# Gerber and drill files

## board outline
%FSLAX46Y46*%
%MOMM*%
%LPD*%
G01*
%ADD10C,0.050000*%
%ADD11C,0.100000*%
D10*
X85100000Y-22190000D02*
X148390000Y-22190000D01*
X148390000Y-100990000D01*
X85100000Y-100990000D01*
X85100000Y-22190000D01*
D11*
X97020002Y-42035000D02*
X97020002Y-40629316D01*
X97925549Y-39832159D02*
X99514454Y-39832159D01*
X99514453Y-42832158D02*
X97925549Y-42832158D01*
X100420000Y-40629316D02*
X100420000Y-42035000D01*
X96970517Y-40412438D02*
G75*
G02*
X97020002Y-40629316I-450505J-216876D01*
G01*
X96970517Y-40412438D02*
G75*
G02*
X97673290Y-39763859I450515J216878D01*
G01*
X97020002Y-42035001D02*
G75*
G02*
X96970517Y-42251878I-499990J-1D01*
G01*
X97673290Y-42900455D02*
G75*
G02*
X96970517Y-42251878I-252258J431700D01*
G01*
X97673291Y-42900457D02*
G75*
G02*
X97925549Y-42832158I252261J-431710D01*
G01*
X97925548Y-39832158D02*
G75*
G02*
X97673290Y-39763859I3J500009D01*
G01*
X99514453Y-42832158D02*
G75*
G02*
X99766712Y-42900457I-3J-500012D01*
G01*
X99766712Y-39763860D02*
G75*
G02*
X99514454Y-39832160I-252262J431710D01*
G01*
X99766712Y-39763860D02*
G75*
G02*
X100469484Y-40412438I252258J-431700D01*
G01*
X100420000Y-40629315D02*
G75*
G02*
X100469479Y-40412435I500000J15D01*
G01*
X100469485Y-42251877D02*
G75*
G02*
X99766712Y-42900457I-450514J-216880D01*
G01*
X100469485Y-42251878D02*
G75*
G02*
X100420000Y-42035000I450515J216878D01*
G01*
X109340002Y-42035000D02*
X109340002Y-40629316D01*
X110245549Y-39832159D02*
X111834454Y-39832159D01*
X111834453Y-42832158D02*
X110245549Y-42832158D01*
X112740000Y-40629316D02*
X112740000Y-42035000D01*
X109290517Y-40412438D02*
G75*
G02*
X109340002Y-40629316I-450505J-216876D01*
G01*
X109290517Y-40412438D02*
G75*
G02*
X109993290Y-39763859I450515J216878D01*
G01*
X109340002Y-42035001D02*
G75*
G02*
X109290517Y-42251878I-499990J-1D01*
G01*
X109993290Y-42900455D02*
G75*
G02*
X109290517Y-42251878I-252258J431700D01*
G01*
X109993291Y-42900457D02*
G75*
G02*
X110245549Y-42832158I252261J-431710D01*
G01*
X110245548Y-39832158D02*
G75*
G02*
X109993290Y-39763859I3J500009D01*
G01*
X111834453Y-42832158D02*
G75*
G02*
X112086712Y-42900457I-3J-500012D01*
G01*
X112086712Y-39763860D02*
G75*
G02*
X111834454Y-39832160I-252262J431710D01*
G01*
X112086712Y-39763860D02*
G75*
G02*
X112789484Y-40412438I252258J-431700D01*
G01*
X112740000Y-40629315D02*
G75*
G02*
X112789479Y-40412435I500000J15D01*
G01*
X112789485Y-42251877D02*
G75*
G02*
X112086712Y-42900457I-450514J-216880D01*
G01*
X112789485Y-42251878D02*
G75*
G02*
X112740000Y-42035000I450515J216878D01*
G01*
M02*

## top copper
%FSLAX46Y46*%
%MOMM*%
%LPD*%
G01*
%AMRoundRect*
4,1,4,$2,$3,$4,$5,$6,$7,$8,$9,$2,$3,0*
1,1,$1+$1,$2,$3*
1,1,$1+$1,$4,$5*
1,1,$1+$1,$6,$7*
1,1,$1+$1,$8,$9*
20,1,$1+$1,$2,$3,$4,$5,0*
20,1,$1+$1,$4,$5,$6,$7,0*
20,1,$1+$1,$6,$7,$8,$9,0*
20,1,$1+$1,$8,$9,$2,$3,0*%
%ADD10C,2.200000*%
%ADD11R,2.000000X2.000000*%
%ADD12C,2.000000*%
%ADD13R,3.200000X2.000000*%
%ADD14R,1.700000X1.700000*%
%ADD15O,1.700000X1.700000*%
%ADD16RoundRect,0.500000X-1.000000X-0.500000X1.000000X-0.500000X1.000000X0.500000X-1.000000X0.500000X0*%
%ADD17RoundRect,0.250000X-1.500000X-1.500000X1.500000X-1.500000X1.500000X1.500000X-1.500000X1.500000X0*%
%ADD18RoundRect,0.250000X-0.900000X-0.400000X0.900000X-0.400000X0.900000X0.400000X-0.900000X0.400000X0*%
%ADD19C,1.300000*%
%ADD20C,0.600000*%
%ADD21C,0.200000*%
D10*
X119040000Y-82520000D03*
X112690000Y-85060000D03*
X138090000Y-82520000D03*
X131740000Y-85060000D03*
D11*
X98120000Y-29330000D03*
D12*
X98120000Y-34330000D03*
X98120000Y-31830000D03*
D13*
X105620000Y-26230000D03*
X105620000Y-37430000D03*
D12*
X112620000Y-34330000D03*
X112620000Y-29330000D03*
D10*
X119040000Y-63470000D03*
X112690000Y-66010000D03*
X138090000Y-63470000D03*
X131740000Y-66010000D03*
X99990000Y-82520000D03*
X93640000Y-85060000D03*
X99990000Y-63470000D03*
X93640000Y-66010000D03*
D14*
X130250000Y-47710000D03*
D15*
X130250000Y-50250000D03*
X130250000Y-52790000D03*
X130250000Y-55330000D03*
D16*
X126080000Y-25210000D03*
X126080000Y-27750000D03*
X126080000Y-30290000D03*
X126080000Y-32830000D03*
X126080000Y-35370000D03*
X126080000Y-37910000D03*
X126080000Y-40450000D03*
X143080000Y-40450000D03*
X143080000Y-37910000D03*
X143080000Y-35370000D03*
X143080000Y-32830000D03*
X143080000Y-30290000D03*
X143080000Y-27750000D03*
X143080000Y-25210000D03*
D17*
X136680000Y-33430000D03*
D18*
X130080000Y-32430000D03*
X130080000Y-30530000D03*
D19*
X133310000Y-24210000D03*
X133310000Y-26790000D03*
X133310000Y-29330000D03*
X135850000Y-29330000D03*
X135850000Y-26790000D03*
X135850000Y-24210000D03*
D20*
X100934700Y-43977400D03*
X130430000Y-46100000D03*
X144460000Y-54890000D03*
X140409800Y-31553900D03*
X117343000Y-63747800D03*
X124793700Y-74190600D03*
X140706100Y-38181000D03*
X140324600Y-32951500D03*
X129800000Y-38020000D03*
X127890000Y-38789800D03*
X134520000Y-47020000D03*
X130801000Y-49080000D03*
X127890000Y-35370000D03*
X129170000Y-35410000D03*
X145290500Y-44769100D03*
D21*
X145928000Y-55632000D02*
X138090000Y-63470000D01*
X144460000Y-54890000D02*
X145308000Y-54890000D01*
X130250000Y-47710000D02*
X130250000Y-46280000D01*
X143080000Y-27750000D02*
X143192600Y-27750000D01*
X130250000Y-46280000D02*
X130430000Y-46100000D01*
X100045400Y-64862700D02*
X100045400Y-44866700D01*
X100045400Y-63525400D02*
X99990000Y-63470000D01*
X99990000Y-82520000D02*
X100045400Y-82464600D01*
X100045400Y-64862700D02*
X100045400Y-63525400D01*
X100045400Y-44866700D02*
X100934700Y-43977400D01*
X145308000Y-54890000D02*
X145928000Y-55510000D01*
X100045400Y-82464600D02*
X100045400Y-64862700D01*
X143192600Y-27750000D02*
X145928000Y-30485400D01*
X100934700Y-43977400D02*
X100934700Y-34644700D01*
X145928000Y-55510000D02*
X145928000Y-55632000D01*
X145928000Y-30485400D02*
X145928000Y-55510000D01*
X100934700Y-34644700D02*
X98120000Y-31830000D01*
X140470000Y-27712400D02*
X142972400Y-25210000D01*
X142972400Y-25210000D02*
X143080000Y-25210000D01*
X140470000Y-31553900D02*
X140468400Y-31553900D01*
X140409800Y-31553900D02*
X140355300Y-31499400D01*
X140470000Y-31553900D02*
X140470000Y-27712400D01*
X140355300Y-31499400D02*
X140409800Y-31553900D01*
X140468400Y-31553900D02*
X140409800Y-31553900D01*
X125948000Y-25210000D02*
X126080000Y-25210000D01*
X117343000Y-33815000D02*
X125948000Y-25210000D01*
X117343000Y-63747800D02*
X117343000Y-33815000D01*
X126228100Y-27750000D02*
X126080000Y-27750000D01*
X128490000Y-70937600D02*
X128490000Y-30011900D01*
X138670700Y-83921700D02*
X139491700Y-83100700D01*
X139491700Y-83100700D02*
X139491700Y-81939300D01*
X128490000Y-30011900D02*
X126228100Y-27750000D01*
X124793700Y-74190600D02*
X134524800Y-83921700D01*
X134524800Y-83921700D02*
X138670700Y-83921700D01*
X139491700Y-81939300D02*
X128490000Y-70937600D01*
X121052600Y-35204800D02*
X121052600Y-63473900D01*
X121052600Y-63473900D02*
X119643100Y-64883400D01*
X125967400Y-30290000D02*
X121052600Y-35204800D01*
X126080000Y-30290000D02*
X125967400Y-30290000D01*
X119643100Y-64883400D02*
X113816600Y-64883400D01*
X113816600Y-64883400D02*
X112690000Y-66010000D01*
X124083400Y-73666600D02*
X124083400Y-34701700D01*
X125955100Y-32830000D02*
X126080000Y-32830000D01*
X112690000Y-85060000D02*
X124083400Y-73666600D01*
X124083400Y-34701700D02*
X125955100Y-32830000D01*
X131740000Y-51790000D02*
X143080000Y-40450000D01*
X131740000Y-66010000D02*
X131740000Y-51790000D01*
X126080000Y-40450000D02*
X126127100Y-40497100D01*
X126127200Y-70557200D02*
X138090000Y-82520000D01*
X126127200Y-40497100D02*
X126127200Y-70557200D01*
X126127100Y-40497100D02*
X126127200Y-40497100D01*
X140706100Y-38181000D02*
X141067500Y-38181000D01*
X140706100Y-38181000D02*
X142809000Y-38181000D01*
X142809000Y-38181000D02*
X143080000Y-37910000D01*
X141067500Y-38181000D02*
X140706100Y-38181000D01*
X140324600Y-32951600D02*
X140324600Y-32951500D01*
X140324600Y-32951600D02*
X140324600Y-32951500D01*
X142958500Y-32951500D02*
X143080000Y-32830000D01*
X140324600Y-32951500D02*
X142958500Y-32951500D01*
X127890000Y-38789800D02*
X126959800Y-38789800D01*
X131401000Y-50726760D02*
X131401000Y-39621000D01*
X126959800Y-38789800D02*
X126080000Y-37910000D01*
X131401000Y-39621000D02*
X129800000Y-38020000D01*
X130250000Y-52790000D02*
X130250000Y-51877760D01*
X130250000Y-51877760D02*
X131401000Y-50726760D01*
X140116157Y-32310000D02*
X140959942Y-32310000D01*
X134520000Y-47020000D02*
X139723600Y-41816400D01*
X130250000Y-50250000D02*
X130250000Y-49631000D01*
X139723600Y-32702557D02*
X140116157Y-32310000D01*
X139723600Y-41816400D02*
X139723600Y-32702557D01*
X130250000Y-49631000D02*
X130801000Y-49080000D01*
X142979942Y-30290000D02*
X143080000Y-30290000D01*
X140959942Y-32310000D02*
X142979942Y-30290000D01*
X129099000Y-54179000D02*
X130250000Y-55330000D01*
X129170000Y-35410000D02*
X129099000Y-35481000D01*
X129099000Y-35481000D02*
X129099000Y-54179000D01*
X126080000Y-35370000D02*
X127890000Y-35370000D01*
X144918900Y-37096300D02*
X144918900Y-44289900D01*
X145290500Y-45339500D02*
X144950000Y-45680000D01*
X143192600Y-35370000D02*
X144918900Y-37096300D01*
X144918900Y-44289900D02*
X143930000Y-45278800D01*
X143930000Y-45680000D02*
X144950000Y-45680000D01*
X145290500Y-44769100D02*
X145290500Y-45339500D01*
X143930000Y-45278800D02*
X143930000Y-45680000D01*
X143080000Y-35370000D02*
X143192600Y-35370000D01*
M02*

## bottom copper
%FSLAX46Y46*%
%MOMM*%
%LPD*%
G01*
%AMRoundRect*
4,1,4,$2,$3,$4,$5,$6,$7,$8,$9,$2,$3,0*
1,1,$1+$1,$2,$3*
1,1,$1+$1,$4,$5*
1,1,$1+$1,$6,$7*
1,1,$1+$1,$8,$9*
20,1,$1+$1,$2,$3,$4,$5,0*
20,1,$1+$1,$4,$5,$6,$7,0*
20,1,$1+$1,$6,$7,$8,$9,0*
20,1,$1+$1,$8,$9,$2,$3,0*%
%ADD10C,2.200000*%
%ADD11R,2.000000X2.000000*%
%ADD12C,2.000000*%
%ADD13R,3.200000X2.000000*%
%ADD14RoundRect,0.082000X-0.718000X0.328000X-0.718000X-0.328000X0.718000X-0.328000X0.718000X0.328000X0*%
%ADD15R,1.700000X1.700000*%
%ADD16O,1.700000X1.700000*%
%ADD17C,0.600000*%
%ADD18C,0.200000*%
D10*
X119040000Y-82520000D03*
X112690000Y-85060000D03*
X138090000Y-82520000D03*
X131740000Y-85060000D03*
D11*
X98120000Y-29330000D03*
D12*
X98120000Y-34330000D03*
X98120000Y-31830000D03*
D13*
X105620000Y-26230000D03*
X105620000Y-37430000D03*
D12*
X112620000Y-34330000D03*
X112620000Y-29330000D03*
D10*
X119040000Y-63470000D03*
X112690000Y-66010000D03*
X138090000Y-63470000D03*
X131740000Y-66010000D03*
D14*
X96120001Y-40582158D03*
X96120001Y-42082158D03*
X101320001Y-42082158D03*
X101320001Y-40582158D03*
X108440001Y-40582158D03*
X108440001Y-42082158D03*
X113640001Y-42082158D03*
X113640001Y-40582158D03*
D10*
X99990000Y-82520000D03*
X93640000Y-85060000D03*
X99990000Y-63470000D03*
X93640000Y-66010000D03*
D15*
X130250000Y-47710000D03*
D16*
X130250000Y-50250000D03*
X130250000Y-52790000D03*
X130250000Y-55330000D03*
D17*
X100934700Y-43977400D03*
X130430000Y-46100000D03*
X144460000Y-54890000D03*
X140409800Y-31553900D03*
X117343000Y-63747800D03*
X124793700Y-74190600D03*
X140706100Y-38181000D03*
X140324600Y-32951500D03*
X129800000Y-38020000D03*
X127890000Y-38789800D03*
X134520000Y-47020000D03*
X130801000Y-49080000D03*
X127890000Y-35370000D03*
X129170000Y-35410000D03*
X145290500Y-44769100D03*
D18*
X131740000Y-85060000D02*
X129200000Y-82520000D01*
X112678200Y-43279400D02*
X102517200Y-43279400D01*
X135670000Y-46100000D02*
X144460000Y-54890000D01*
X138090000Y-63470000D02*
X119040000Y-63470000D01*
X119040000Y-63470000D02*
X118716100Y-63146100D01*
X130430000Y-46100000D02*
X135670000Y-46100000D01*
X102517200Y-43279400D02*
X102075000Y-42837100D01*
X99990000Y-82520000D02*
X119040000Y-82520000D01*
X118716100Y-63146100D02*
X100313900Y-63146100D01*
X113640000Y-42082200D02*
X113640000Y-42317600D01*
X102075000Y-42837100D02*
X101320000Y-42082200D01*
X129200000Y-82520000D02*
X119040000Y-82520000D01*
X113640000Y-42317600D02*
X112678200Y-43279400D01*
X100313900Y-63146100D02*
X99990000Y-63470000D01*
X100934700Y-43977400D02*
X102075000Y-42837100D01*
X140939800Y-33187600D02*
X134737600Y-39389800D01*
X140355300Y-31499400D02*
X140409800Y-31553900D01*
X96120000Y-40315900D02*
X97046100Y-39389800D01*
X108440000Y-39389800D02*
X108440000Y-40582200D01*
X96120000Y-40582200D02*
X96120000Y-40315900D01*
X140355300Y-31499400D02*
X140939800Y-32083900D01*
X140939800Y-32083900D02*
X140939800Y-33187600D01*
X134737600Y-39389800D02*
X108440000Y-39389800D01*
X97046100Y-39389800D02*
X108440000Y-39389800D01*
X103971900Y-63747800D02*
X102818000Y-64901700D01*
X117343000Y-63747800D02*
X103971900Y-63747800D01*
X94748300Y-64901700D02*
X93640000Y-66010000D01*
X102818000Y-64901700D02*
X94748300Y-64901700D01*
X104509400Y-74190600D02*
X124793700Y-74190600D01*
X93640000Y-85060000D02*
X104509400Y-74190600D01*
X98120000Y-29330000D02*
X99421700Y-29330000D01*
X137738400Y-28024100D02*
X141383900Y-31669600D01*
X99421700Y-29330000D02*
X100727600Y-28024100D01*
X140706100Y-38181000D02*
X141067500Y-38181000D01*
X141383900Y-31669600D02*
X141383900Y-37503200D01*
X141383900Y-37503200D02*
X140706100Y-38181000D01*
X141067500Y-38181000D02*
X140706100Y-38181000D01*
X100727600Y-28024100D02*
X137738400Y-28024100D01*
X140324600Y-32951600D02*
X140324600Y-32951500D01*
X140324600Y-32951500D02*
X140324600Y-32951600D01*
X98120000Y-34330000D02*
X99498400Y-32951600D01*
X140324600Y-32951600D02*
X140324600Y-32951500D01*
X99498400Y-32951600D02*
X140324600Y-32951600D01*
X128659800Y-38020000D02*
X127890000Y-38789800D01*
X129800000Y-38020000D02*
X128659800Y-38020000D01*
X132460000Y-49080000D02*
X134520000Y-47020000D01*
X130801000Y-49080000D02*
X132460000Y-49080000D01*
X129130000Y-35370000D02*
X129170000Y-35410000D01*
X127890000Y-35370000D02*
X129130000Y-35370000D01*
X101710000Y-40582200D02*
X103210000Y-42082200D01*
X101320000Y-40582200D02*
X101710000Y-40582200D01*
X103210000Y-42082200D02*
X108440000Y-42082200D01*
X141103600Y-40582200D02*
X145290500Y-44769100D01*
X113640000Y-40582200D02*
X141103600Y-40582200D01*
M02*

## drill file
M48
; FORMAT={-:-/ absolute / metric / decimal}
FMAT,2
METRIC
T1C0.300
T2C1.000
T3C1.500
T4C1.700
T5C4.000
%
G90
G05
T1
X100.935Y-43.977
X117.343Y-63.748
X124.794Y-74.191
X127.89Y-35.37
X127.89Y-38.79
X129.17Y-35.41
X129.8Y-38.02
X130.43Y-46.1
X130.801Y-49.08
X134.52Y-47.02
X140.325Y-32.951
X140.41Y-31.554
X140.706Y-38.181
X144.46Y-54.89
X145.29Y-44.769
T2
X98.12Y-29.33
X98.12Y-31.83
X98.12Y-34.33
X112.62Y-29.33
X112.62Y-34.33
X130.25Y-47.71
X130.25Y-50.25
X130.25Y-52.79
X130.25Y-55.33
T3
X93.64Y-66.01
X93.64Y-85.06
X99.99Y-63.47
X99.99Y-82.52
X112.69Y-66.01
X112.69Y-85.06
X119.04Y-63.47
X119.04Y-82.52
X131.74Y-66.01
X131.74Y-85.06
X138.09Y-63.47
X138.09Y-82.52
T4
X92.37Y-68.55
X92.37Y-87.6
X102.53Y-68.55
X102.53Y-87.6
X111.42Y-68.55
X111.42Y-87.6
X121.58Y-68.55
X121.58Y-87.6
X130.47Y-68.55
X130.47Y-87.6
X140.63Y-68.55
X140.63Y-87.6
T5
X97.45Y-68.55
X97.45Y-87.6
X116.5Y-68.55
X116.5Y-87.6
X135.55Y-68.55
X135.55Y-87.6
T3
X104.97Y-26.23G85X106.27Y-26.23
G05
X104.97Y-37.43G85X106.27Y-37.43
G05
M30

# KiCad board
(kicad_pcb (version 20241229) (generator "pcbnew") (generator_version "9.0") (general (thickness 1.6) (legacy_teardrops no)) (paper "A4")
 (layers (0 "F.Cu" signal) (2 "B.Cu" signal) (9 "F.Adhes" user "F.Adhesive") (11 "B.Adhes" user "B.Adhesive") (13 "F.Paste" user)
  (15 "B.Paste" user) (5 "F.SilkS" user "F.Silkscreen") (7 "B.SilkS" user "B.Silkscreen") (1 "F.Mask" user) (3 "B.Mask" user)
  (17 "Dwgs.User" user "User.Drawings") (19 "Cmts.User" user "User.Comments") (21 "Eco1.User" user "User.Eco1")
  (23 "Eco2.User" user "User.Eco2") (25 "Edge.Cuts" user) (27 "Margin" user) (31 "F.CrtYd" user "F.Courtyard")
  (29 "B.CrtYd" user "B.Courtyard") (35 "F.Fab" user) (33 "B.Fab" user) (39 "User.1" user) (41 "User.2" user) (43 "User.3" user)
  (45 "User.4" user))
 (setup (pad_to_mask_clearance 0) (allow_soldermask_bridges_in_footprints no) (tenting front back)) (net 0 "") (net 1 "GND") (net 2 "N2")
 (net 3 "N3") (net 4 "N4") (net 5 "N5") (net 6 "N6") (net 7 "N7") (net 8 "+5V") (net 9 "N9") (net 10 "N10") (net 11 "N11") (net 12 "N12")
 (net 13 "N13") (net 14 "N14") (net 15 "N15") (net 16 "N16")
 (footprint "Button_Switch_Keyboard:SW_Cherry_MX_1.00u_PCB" (layer "F.Cu") (at 119.04 82.52)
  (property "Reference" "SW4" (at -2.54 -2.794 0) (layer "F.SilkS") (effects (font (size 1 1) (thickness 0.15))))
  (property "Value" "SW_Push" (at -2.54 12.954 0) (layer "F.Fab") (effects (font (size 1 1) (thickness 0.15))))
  (pad "" np_thru_hole circle (at -7.62 5.08) (size 1.7 1.7) (drill 1.7) (layers "*.Cu" "*.Mask"))
  (pad "" np_thru_hole circle (at -2.54 5.08) (size 4 4) (drill 4) (layers "*.Cu" "*.Mask"))
  (pad "" np_thru_hole circle (at 2.54 5.08) (size 1.7 1.7) (drill 1.7) (layers "*.Cu" "*.Mask"))
  (pad "1" thru_hole circle (at 0 0) (size 2.2 2.2) (drill 1.5) (layers "*.Cu" "*.Mask") (remove_unused_layers no) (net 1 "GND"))
  (pad "2" thru_hole circle (at -6.35 2.54) (size 2.2 2.2) (drill 1.5) (layers "*.Cu" "*.Mask") (remove_unused_layers no) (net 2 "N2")))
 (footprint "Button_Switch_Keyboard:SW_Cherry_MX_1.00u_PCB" (layer "F.Cu") (at 138.09 82.52)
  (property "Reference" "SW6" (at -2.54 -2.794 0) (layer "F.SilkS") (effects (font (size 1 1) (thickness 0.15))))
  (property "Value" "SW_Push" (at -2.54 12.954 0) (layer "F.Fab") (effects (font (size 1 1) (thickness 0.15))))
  (pad "" np_thru_hole circle (at -7.62 5.08) (size 1.7 1.7) (drill 1.7) (layers "*.Cu" "*.Mask"))
  (pad "" np_thru_hole circle (at -2.54 5.08) (size 4 4) (drill 4) (layers "*.Cu" "*.Mask"))
  (pad "" np_thru_hole circle (at 2.54 5.08) (size 1.7 1.7) (drill 1.7) (layers "*.Cu" "*.Mask"))
  (pad "1" thru_hole circle (at 0 0) (size 2.2 2.2) (drill 1.5) (layers "*.Cu" "*.Mask") (remove_unused_layers no) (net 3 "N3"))
  (pad "2" thru_hole circle (at -6.35 2.54) (size 2.2 2.2) (drill 1.5) (layers "*.Cu" "*.Mask") (remove_unused_layers no) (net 1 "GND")))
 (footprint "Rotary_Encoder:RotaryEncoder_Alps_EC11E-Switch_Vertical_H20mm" (layer "F.Cu") (at 98.12 29.33)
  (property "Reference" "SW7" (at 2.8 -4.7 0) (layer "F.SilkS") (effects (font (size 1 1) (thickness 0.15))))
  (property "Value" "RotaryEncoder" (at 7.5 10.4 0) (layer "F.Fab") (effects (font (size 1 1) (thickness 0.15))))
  (pad "A" thru_hole rect (at 0 0) (size 2 2) (drill 1) (layers "*.Cu" "*.Mask") (remove_unused_layers no) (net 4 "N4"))
  (pad "B" thru_hole circle (at 0 5) (size 2 2) (drill 1) (layers "*.Cu" "*.Mask") (remove_unused_layers no) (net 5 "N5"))
  (pad "C" thru_hole circle (at 0 2.5) (size 2 2) (drill 1) (layers "*.Cu" "*.Mask") (remove_unused_layers no) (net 1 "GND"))
  (pad "MP" thru_hole rect (at 7.5 -3.1) (size 3.2 2) (drill oval 2.8 1.5) (layers "*.Cu" "*.Mask") (remove_unused_layers no))
  (pad "MP" thru_hole rect (at 7.5 8.1) (size 3.2 2) (drill oval 2.8 1.5) (layers "*.Cu" "*.Mask") (remove_unused_layers no))
  (pad "S1" thru_hole circle (at 14.5 5) (size 2 2) (drill 1) (layers "*.Cu" "*.Mask") (remove_unused_layers no))
  (pad "S2" thru_hole circle (at 14.5 0) (size 2 2) (drill 1) (layers "*.Cu" "*.Mask") (remove_unused_layers no)))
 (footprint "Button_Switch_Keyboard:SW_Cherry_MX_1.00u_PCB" (layer "F.Cu") (at 119.04 63.47)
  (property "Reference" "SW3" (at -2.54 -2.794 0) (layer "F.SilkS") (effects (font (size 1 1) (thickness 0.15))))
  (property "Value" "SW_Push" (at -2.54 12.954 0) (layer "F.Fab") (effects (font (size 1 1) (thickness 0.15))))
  (pad "" np_thru_hole circle (at -7.62 5.08) (size 1.7 1.7) (drill 1.7) (layers "*.Cu" "*.Mask"))
  (pad "" np_thru_hole circle (at -2.54 5.08) (size 4 4) (drill 4) (layers "*.Cu" "*.Mask"))
  (pad "" np_thru_hole circle (at 2.54 5.08) (size 1.7 1.7) (drill 1.7) (layers "*.Cu" "*.Mask"))
  (pad "1" thru_hole circle (at 0 0) (size 2.2 2.2) (drill 1.5) (layers "*.Cu" "*.Mask") (remove_unused_layers no) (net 1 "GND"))
  (pad "2" thru_hole circle (at -6.35 2.54) (size 2.2 2.2) (drill 1.5) (layers "*.Cu" "*.Mask") (remove_unused_layers no) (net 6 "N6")))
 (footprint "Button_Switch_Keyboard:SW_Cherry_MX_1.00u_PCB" (layer "F.Cu") (at 138.09 63.47)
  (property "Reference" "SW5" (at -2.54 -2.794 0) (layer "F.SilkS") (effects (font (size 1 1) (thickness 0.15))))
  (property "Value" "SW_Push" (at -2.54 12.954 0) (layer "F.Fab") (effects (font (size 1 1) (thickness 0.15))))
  (pad "" np_thru_hole circle (at -7.62 5.08) (size 1.7 1.7) (drill 1.7) (layers "*.Cu" "*.Mask"))
  (pad "" np_thru_hole circle (at -2.54 5.08) (size 4 4) (drill 4) (layers "*.Cu" "*.Mask"))
  (pad "" np_thru_hole circle (at 2.54 5.08) (size 1.7 1.7) (drill 1.7) (layers "*.Cu" "*.Mask"))
  (pad "1" thru_hole circle (at 0 0) (size 2.2 2.2) (drill 1.5) (layers "*.Cu" "*.Mask") (remove_unused_layers no) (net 1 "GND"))
  (pad "2" thru_hole circle (at -6.35 2.54) (size 2.2 2.2) (drill 1.5) (layers "*.Cu" "*.Mask") (remove_unused_layers no) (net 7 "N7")))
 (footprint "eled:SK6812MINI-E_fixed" (layer "F.Cu") (at 98.72 41.435)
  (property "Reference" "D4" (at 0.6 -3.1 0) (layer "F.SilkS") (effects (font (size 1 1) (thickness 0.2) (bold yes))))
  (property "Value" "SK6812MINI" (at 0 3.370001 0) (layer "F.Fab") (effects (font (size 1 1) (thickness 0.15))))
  (fp_line (start -1.699998 0.6) (end -1.699998 -0.805684) (stroke (width 0.1) (type solid)) (layer "Edge.Cuts"))
  (fp_line (start -0.794451 -1.602841) (end 0.794454 -1.602841) (stroke (width 0.1) (type solid)) (layer "Edge.Cuts"))
  (fp_line (start 0.794453 1.397158) (end -0.794451 1.397158) (stroke (width 0.1) (type solid)) (layer "Edge.Cuts"))
  (fp_line (start 1.7 -0.805684) (end 1.7 0.6) (stroke (width 0.1) (type solid)) (layer "Edge.Cuts"))
  (fp_arc (start -1.749483 -1.022562) (mid -1.712526 -0.91691) (end -1.699998 -0.805684) (stroke (width 0.1) (type solid))
   (layer "Edge.Cuts"))
  (fp_arc (start -1.749483 -1.022562) (mid -1.63807 -1.606877) (end -1.04671 -1.671141) (stroke (width 0.1) (type solid))
   (layer "Edge.Cuts"))
  (fp_arc (start -1.699998 0.600001) (mid -1.712526 0.711226) (end -1.749483 0.816878) (stroke (width 0.1) (type solid)) (layer "Edge.Cuts"))
  (fp_arc (start -1.04671 1.465455) (mid -1.638069 1.401192) (end -1.749483 0.816878) (stroke (width 0.1) (type solid)) (layer "Edge.Cuts"))
  (fp_arc (start -1.046709 1.465457) (mid -0.925121 1.414535) (end -0.794451 1.397158) (stroke (width 0.1) (type solid)) (layer "Edge.Cuts"))
  (fp_arc (start -0.794452 -1.602842) (mid -0.925122 -1.620219) (end -1.04671 -1.671141) (stroke (width 0.1) (type solid))
   (layer "Edge.Cuts"))
  (fp_arc (start 0.794453 1.397158) (mid 0.925124 1.414535) (end 1.046712 1.465457) (stroke (width 0.1) (type solid)) (layer "Edge.Cuts"))
  (fp_arc (start 1.046712 -1.67114) (mid 0.925124 -1.620218) (end 0.794454 -1.602841) (stroke (width 0.1) (type solid)) (layer "Edge.Cuts"))
  (fp_arc (start 1.046712 -1.67114) (mid 1.638072 -1.606876) (end 1.749485 -1.022562) (stroke (width 0.1) (type solid)) (layer "Edge.Cuts"))
  (fp_arc (start 1.7 -0.805685) (mid 1.712528 -0.91691) (end 1.749485 -1.022562) (stroke (width 0.1) (type solid)) (layer "Edge.Cuts"))
  (fp_arc (start 1.749485 0.816877) (mid 1.638073 1.401193) (end 1.046712 1.465457) (stroke (width 0.1) (type solid)) (layer "Edge.Cuts"))
  (fp_arc (start 1.749485 0.816878) (mid 1.712528 0.711226) (end 1.7 0.6) (stroke (width 0.1) (type solid)) (layer "Edge.Cuts"))
  (pad "1" smd roundrect (at -2.599999 -0.852842 270) (size 0.82 1.6) (layers "B.Cu" "B.Mask" "B.Paste") (roundrect_rratio 0.1)
   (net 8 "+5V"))
  (pad "2" smd roundrect (at -2.599999 0.647158 270) (size 0.82 1.6) (layers "B.Cu" "B.Mask" "B.Paste") (roundrect_rratio 0.1) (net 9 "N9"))
  (pad "3" smd roundrect (at 2.600001 0.647158 270) (size 0.82 1.6) (layers "B.Cu" "B.Mask" "B.Paste") (roundrect_rratio 0.1) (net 1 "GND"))
  (pad "4" smd roundrect (at 2.600001 -0.852842 270) (size 0.82 1.6) (layers "B.Cu" "B.Mask" "B.Paste") (roundrect_rratio 0.1)
   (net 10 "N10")))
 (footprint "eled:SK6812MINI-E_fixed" (layer "F.Cu") (at 111.04 41.435)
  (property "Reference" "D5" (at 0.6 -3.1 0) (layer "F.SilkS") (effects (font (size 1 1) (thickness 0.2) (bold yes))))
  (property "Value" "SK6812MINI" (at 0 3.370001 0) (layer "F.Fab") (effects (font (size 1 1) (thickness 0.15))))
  (fp_line (start -1.699998 0.6) (end -1.699998 -0.805684) (stroke (width 0.1) (type solid)) (layer "Edge.Cuts"))
  (fp_line (start -0.794451 -1.602841) (end 0.794454 -1.602841) (stroke (width 0.1) (type solid)) (layer "Edge.Cuts"))
  (fp_line (start 0.794453 1.397158) (end -0.794451 1.397158) (stroke (width 0.1) (type solid)) (layer "Edge.Cuts"))
  (fp_line (start 1.7 -0.805684) (end 1.7 0.6) (stroke (width 0.1) (type solid)) (layer "Edge.Cuts"))
  (fp_arc (start -1.749483 -1.022562) (mid -1.712526 -0.91691) (end -1.699998 -0.805684) (stroke (width 0.1) (type solid))
   (layer "Edge.Cuts"))
  (fp_arc (start -1.749483 -1.022562) (mid -1.63807 -1.606877) (end -1.04671 -1.671141) (stroke (width 0.1) (type solid))
   (layer "Edge.Cuts"))
  (fp_arc (start -1.699998 0.600001) (mid -1.712526 0.711226) (end -1.749483 0.816878) (stroke (width 0.1) (type solid)) (layer "Edge.Cuts"))
  (fp_arc (start -1.04671 1.465455) (mid -1.638069 1.401192) (end -1.749483 0.816878) (stroke (width 0.1) (type solid)) (layer "Edge.Cuts"))
  (fp_arc (start -1.046709 1.465457) (mid -0.925121 1.414535) (end -0.794451 1.397158) (stroke (width 0.1) (type solid)) (layer "Edge.Cuts"))
  (fp_arc (start -0.794452 -1.602842) (mid -0.925122 -1.620219) (end -1.04671 -1.671141) (stroke (width 0.1) (type solid))
   (layer "Edge.Cuts"))
  (fp_arc (start 0.794453 1.397158) (mid 0.925124 1.414535) (end 1.046712 1.465457) (stroke (width 0.1) (type solid)) (layer "Edge.Cuts"))
  (fp_arc (start 1.046712 -1.67114) (mid 0.925124 -1.620218) (end 0.794454 -1.602841) (stroke (width 0.1) (type solid)) (layer "Edge.Cuts"))
  (fp_arc (start 1.046712 -1.67114) (mid 1.638072 -1.606876) (end 1.749485 -1.022562) (stroke (width 0.1) (type solid)) (layer "Edge.Cuts"))
  (fp_arc (start 1.7 -0.805685) (mid 1.712528 -0.91691) (end 1.749485 -1.022562) (stroke (width 0.1) (type solid)) (layer "Edge.Cuts"))
  (fp_arc (start 1.749485 0.816877) (mid 1.638073 1.401193) (end 1.046712 1.465457) (stroke (width 0.1) (type solid)) (layer "Edge.Cuts"))
  (fp_arc (start 1.749485 0.816878) (mid 1.712528 0.711226) (end 1.7 0.6) (stroke (width 0.1) (type solid)) (layer "Edge.Cuts"))
  (pad "1" smd roundrect (at -2.599999 -0.852842 270) (size 0.82 1.6) (layers "B.Cu" "B.Mask" "B.Paste") (roundrect_rratio 0.1)
   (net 8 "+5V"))
  (pad "2" smd roundrect (at -2.599999 0.647158 270) (size 0.82 1.6) (layers "B.Cu" "B.Mask" "B.Paste") (roundrect_rratio 0.1)
   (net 10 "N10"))
  (pad "3" smd roundrect (at 2.600001 0.647158 270) (size 0.82 1.6) (layers "B.Cu" "B.Mask" "B.Paste") (roundrect_rratio 0.1) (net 1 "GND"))
  (pad "4" smd roundrect (at 2.600001 -0.852842 270) (size 0.82 1.6) (layers "B.Cu" "B.Mask" "B.Paste") (roundrect_rratio 0.1)
   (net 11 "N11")))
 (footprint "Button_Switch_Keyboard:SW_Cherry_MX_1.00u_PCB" (layer "F.Cu") (at 99.99 82.52)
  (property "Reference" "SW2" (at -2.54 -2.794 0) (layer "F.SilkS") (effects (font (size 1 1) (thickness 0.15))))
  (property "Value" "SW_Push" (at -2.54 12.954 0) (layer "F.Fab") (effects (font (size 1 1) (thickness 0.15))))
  (pad "" np_thru_hole circle (at -7.62 5.08) (size 1.7 1.7) (drill 1.7) (layers "*.Cu" "*.Mask"))
  (pad "" np_thru_hole circle (at -2.54 5.08) (size 4 4) (drill 4) (layers "*.Cu" "*.Mask"))
  (pad "" np_thru_hole circle (at 2.54 5.08) (size 1.7 1.7) (drill 1.7) (layers "*.Cu" "*.Mask"))
  (pad "1" thru_hole circle (at 0 0) (size 2.2 2.2) (drill 1.5) (layers "*.Cu" "*.Mask") (remove_unused_layers no) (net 1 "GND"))
  (pad "2" thru_hole circle (at -6.35 2.54) (size 2.2 2.2) (drill 1.5) (layers "*.Cu" "*.Mask") (remove_unused_layers no) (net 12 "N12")))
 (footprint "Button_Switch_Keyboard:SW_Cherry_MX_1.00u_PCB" (layer "F.Cu") (at 99.99 63.47)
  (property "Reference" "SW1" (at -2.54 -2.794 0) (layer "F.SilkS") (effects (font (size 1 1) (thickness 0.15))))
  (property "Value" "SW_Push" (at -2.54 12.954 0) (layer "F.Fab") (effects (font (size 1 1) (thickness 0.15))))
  (pad "" np_thru_hole circle (at -7.62 5.08) (size 1.7 1.7) (drill 1.7) (layers "*.Cu" "*.Mask"))
  (pad "" np_thru_hole circle (at -2.54 5.08) (size 4 4) (drill 4) (layers "*.Cu" "*.Mask"))
  (pad "" np_thru_hole circle (at 2.54 5.08) (size 1.7 1.7) (drill 1.7) (layers "*.Cu" "*.Mask"))
  (pad "1" thru_hole circle (at 0 0) (size 2.2 2.2) (drill 1.5) (layers "*.Cu" "*.Mask") (remove_unused_layers no) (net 1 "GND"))
  (pad "2" thru_hole circle (at -6.35 2.54) (size 2.2 2.2) (drill 1.5) (layers "*.Cu" "*.Mask") (remove_unused_layers no) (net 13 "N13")))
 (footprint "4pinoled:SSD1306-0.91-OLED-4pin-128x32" (layer "F.Cu") (at 93.75 45.52)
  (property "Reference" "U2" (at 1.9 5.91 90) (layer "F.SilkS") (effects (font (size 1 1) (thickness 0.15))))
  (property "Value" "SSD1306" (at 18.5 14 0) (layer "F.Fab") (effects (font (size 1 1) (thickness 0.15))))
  (pad "1" thru_hole rect (at 36.5 2.19) (size 1.7 1.7) (drill 1) (layers "*.Cu" "*.Mask") (remove_unused_layers no) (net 1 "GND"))
  (pad "2" thru_hole oval (at 36.5 4.73) (size 1.7 1.7) (drill 1) (layers "*.Cu" "*.Mask") (remove_unused_layers no) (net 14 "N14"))
  (pad "3" thru_hole oval (at 36.5 7.27) (size 1.7 1.7) (drill 1) (layers "*.Cu" "*.Mask") (remove_unused_layers no) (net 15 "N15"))
  (pad "4" thru_hole oval (at 36.5 9.81) (size 1.7 1.7) (drill 1) (layers "*.Cu" "*.Mask") (remove_unused_layers no) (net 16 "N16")))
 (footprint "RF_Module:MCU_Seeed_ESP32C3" (layer "F.Cu") (at 134.58 32.83)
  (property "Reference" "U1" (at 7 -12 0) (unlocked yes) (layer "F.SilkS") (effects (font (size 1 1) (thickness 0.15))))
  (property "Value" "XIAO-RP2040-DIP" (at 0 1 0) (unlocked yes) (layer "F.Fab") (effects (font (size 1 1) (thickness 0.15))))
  (pad "" smd roundrect (at 1.1 -0.4) (size 1.5 1.5) (layers "F.Paste") (roundrect_rratio 0.1666666667))
  (pad "" smd roundrect (at 1.1 1.6) (size 1.5 1.5) (layers "F.Paste") (roundrect_rratio 0.1666666667))
  (pad "" smd roundrect (at 3.1 -0.4) (size 1.5 1.5) (layers "F.Paste") (roundrect_rratio 0.1666666667))
  (pad "" smd roundrect (at 3.1 1.6) (size 1.5 1.5) (layers "F.Paste") (roundrect_rratio 0.1666666667))
  (pad "1" smd roundrect (at -8.5 -7.62) (size 3 2) (layers "F.Cu" "F.Mask" "F.Paste") (roundrect_rratio 0.25) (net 13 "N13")
   (thermal_bridge_angle 45))
  (pad "2" smd roundrect (at -8.5 -5.08) (size 3 2) (layers "F.Cu" "F.Mask" "F.Paste") (roundrect_rratio 0.25) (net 12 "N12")
   (thermal_bridge_angle 45))
  (pad "3" smd roundrect (at -8.5 -2.54) (size 3 2) (layers "F.Cu" "F.Mask" "F.Paste") (roundrect_rratio 0.25) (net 6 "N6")
   (thermal_bridge_angle 45))
  (pad "4" smd roundrect (at -8.5 0) (size 3 2) (layers "F.Cu" "F.Mask" "F.Paste") (roundrect_rratio 0.25) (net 2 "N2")
   (thermal_bridge_angle 45))
  (pad "5" smd roundrect (at -8.5 2.54) (size 3 2) (layers "F.Cu" "F.Mask" "F.Paste") (roundrect_rratio 0.25) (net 16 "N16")
   (thermal_bridge_angle 45))
  (pad "6" smd roundrect (at -8.5 5.08) (size 3 2) (layers "F.Cu" "F.Mask" "F.Paste") (roundrect_rratio 0.25) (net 15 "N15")
   (thermal_bridge_angle 45))
  (pad "7" smd roundrect (at -8.5 7.62) (size 3 2) (layers "F.Cu" "F.Mask" "F.Paste") (roundrect_rratio 0.25) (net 3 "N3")
   (thermal_bridge_angle 45))
  (pad "8" smd roundrect (at 8.5 7.62) (size 3 2) (layers "F.Cu" "F.Mask" "F.Paste") (roundrect_rratio 0.25) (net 7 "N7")
   (thermal_bridge_angle 45))
  (pad "9" smd roundrect (at 8.5 5.08) (size 3 2) (layers "F.Cu" "F.Mask" "F.Paste") (roundrect_rratio 0.25) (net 4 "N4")
   (thermal_bridge_angle 45))
  (pad "10" smd roundrect (at 8.5 2.54) (size 3 2) (layers "F.Cu" "F.Mask" "F.Paste") (roundrect_rratio 0.25) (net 11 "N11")
   (thermal_bridge_angle 45))
  (pad "11" smd roundrect (at 8.5 0) (size 3 2) (layers "F.Cu" "F.Mask" "F.Paste") (roundrect_rratio 0.25) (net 5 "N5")
   (thermal_bridge_angle 45))
  (pad "12" smd roundrect (at 8.5 -2.54) (size 3 2) (layers "F.Cu" "F.Mask" "F.Paste") (roundrect_rratio 0.25) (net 14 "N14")
   (thermal_bridge_angle 45))
  (pad "13" smd roundrect (at 8.5 -5.08) (size 3 2) (layers "F.Cu" "F.Mask" "F.Paste") (roundrect_rratio 0.25) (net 1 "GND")
   (thermal_bridge_angle 45))
  (pad "14" smd roundrect (at 8.5 -7.62) (size 3 2) (layers "F.Cu" "F.Mask" "F.Paste") (roundrect_rratio 0.25) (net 8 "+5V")
   (thermal_bridge_angle 45))
  (pad "15" smd roundrect (at 2.1 0.6) (size 3.5 3.5) (layers "F.Cu" "F.Mask") (roundrect_rratio 0.07142857143))
  (pad "16" smd roundrect (at -4.5 -0.4) (size 2.3 1.3) (layers "F.Cu" "F.Mask" "F.Paste") (roundrect_rratio 0.1923076923))
  (pad "17" smd roundrect (at -4.5 -2.3) (size 2.3 1.3) (layers "F.Cu" "F.Mask" "F.Paste") (roundrect_rratio 0.1923076923))
  (pad "18" smd circle (at -1.27 -8.62) (size 1.3 1.3) (layers "F.Cu" "F.Mask" "F.Paste"))
  (pad "19" smd circle (at -1.27 -6.04) (size 1.3 1.3) (layers "F.Cu" "F.Mask" "F.Paste"))
  (pad "20" smd circle (at -1.27 -3.5) (size 1.3 1.3) (layers "F.Cu" "F.Mask" "F.Paste"))
  (pad "21" smd circle (at 1.27 -3.5) (size 1.3 1.3) (layers "F.Cu" "F.Mask" "F.Paste"))
  (pad "22" smd circle (at 1.27 -6.04) (size 1.3 1.3) (layers "F.Cu" "F.Mask" "F.Paste"))
  (pad "23" smd circle (at 1.27 -8.62) (size 1.3 1.3) (layers "F.Cu" "F.Mask" "F.Paste")))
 (gr_rect (start 85.1 22.19) (end 148.39 100.99) (stroke (width 0.05) (type default)) (fill no) (layer "Edge.Cuts"))
 (segment (start 145.928 55.632) (end 138.09 63.47) (width 0.2) (layer "F.Cu") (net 1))
 (segment (start 144.46 54.89) (end 145.308 54.89) (width 0.2) (layer "F.Cu") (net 1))
 (segment (start 130.25 47.71) (end 130.25 46.28) (width 0.2) (layer "F.Cu") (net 1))
 (segment (start 143.08 27.75) (end 143.1926 27.75) (width 0.2) (layer "F.Cu") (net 1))
 (segment (start 130.25 46.28) (end 130.43 46.1) (width 0.2) (layer "F.Cu") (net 1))
 (segment (start 100.0454 64.8627) (end 100.0454 44.8667) (width 0.2) (layer "F.Cu") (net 1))
 (segment (start 100.0454 63.5254) (end 99.99 63.47) (width 0.2) (layer "F.Cu") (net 1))
 (segment (start 99.99 82.52) (end 100.0454 82.4646) (width 0.2) (layer "F.Cu") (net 1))
 (segment (start 100.0454 64.8627) (end 100.0454 63.5254) (width 0.2) (layer "F.Cu") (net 1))
 (segment (start 100.0454 44.8667) (end 100.9347 43.9774) (width 0.2) (layer "F.Cu") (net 1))
 (segment (start 145.308 54.89) (end 145.928 55.51) (width 0.2) (layer "F.Cu") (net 1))
 (segment (start 100.0454 82.4646) (end 100.0454 64.8627) (width 0.2) (layer "F.Cu") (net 1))
 (segment (start 143.1926 27.75) (end 145.928 30.4854) (width 0.2) (layer "F.Cu") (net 1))
 (segment (start 100.9347 43.9774) (end 100.9347 34.6447) (width 0.2) (layer "F.Cu") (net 1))
 (segment (start 145.928 55.51) (end 145.928 55.632) (width 0.2) (layer "F.Cu") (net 1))
 (segment (start 145.928 30.4854) (end 145.928 55.51) (width 0.2) (layer "F.Cu") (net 1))
 (segment (start 100.9347 34.6447) (end 98.12 31.83) (width 0.2) (layer "F.Cu") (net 1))
 (via (at 100.9347 43.9774) (size 0.6) (drill 0.3) (layers "F.Cu" "B.Cu") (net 1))
 (via (at 130.43 46.1) (size 0.6) (drill 0.3) (layers "F.Cu" "B.Cu") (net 1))
 (via (at 144.46 54.89) (size 0.6) (drill 0.3) (layers "F.Cu" "B.Cu") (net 1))
 (segment (start 131.74 85.06) (end 129.2 82.52) (width 0.2) (layer "B.Cu") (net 1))
 (segment (start 112.6782 43.2794) (end 102.5172 43.2794) (width 0.2) (layer "B.Cu") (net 1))
 (segment (start 135.67 46.1) (end 144.46 54.89) (width 0.2) (layer "B.Cu") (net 1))
 (segment (start 138.09 63.47) (end 119.04 63.47) (width 0.2) (layer "B.Cu") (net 1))
 (segment (start 119.04 63.47) (end 118.7161 63.1461) (width 0.2) (layer "B.Cu") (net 1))
 (segment (start 130.43 46.1) (end 135.67 46.1) (width 0.2) (layer "B.Cu") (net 1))
 (segment (start 102.5172 43.2794) (end 102.075 42.8371) (width 0.2) (layer "B.Cu") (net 1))
 (segment (start 99.99 82.52) (end 119.04 82.52) (width 0.2) (layer "B.Cu") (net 1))
 (segment (start 118.7161 63.1461) (end 100.3139 63.1461) (width 0.2) (layer "B.Cu") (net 1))
 (segment (start 113.64 42.0822) (end 113.64 42.3176) (width 0.2) (layer "B.Cu") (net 1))
 (segment (start 102.075 42.8371) (end 101.32 42.0822) (width 0.2) (layer "B.Cu") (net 1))
 (segment (start 129.2 82.52) (end 119.04 82.52) (width 0.2) (layer "B.Cu") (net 1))
 (segment (start 113.64 42.3176) (end 112.6782 43.2794) (width 0.2) (layer "B.Cu") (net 1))
 (segment (start 100.3139 63.1461) (end 99.99 63.47) (width 0.2) (layer "B.Cu") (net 1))
 (segment (start 100.9347 43.9774) (end 102.075 42.8371) (width 0.2) (layer "B.Cu") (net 1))
 (segment (start 140.47 27.7124) (end 142.9724 25.21) (width 0.2) (layer "F.Cu") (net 8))
 (segment (start 142.9724 25.21) (end 143.08 25.21) (width 0.2) (layer "F.Cu") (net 8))
 (segment (start 140.47 31.5539) (end 140.4684 31.5539) (width 0.2) (layer "F.Cu") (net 8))
 (segment (start 140.4098 31.5539) (end 140.3553 31.4994) (width 0.2) (layer "F.Cu") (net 8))
 (segment (start 140.47 31.5539) (end 140.47 27.7124) (width 0.2) (layer "F.Cu") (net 8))
 (segment (start 140.3553 31.4994) (end 140.4098 31.5539) (width 0.2) (layer "F.Cu") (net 8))
 (segment (start 140.4684 31.5539) (end 140.4098 31.5539) (width 0.2) (layer "F.Cu") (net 8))
 (via (at 140.4098 31.5539) (size 0.6) (drill 0.3) (layers "F.Cu" "B.Cu") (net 8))
 (segment (start 140.9398 33.1876) (end 134.7376 39.3898) (width 0.2) (layer "B.Cu") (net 8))
 (segment (start 140.3553 31.4994) (end 140.4098 31.5539) (width 0.2) (layer "B.Cu") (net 8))
 (segment (start 96.12 40.3159) (end 97.0461 39.3898) (width 0.2) (layer "B.Cu") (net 8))
 (segment (start 108.44 39.3898) (end 108.44 40.5822) (width 0.2) (layer "B.Cu") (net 8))
 (segment (start 96.12 40.5822) (end 96.12 40.3159) (width 0.2) (layer "B.Cu") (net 8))
 (segment (start 140.3553 31.4994) (end 140.9398 32.0839) (width 0.2) (layer "B.Cu") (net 8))
 (segment (start 140.9398 32.0839) (end 140.9398 33.1876) (width 0.2) (layer "B.Cu") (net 8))
 (segment (start 134.7376 39.3898) (end 108.44 39.3898) (width 0.2) (layer "B.Cu") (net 8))
 (segment (start 97.0461 39.3898) (end 108.44 39.3898) (width 0.2) (layer "B.Cu") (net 8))
 (segment (start 125.948 25.21) (end 126.08 25.21) (width 0.2) (layer "F.Cu") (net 13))
 (segment (start 117.343 33.815) (end 125.948 25.21) (width 0.2) (layer "F.Cu") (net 13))
 (segment (start 117.343 63.7478) (end 117.343 33.815) (width 0.2) (layer "F.Cu") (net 13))
 (via (at 117.343 63.7478) (size 0.6) (drill 0.3) (layers "F.Cu" "B.Cu") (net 13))
 (segment (start 103.9719 63.7478) (end 102.818 64.9017) (width 0.2) (layer "B.Cu") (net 13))
 (segment (start 117.343 63.7478) (end 103.9719 63.7478) (width 0.2) (layer "B.Cu") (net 13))
 (segment (start 94.7483 64.9017) (end 93.64 66.01) (width 0.2) (layer "B.Cu") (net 13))
 (segment (start 102.818 64.9017) (end 94.7483 64.9017) (width 0.2) (layer "B.Cu") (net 13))
 (segment (start 126.2281 27.75) (end 126.08 27.75) (width 0.2) (layer "F.Cu") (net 12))
 (segment (start 128.49 70.9376) (end 128.49 30.0119) (width 0.2) (layer "F.Cu") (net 12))
 (segment (start 138.6707 83.9217) (end 139.4917 83.1007) (width 0.2) (layer "F.Cu") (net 12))
 (segment (start 139.4917 83.1007) (end 139.4917 81.9393) (width 0.2) (layer "F.Cu") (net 12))
 (segment (start 128.49 30.0119) (end 126.2281 27.75) (width 0.2) (layer "F.Cu") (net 12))
 (segment (start 124.7937 74.1906) (end 134.5248 83.9217) (width 0.2) (layer "F.Cu") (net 12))
 (segment (start 134.5248 83.9217) (end 138.6707 83.9217) (width 0.2) (layer "F.Cu") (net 12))
 (segment (start 139.4917 81.9393) (end 128.49 70.9376) (width 0.2) (layer "F.Cu") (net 12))
 (via (at 124.7937 74.1906) (size 0.6) (drill 0.3) (layers "F.Cu" "B.Cu") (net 12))
 (segment (start 104.5094 74.1906) (end 124.7937 74.1906) (width 0.2) (layer "B.Cu") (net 12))
 (segment (start 93.64 85.06) (end 104.5094 74.1906) (width 0.2) (layer "B.Cu") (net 12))
 (segment (start 121.0526 35.2048) (end 121.0526 63.4739) (width 0.2) (layer "F.Cu") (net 6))
 (segment (start 121.0526 63.4739) (end 119.6431 64.8834) (width 0.2) (layer "F.Cu") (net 6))
 (segment (start 125.9674 30.29) (end 121.0526 35.2048) (width 0.2) (layer "F.Cu") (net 6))
 (segment (start 126.08 30.29) (end 125.9674 30.29) (width 0.2) (layer "F.Cu") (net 6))
 (segment (start 119.6431 64.8834) (end 113.8166 64.8834) (width 0.2) (layer "F.Cu") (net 6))
 (segment (start 113.8166 64.8834) (end 112.69 66.01) (width 0.2) (layer "F.Cu") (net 6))
 (segment (start 124.0834 73.6666) (end 124.0834 34.7017) (width 0.2) (layer "F.Cu") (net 2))
 (segment (start 125.9551 32.83) (end 126.08 32.83) (width 0.2) (layer "F.Cu") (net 2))
 (segment (start 112.69 85.06) (end 124.0834 73.6666) (width 0.2) (layer "F.Cu") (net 2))
 (segment (start 124.0834 34.7017) (end 125.9551 32.83) (width 0.2) (layer "F.Cu") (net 2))
 (segment (start 131.74 51.79) (end 143.08 40.45) (width 0.2) (layer "F.Cu") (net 7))
 (segment (start 131.74 66.01) (end 131.74 51.79) (width 0.2) (layer "F.Cu") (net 7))
 (segment (start 126.08 40.45) (end 126.1271 40.4971) (width 0.2) (layer "F.Cu") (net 3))
 (segment (start 126.1272 70.5572) (end 138.09 82.52) (width 0.2) (layer "F.Cu") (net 3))
 (segment (start 126.1272 40.4971) (end 126.1272 70.5572) (width 0.2) (layer "F.Cu") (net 3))
 (segment (start 126.1271 40.4971) (end 126.1272 40.4971) (width 0.2) (layer "F.Cu") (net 3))
 (segment (start 140.7061 38.181) (end 141.0675 38.181) (width 0.2) (layer "F.Cu") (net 4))
 (segment (start 140.7061 38.181) (end 142.809 38.181) (width 0.2) (layer "F.Cu") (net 4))
 (segment (start 142.809 38.181) (end 143.08 37.91) (width 0.2) (layer "F.Cu") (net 4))
 (segment (start 141.0675 38.181) (end 140.7061 38.181) (width 0.2) (layer "F.Cu") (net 4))
 (via (at 140.7061 38.181) (size 0.6) (drill 0.3) (layers "F.Cu" "B.Cu") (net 4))
 (segment (start 98.12 29.33) (end 99.4217 29.33) (width 0.2) (layer "B.Cu") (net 4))
 (segment (start 137.7384 28.0241) (end 141.3839 31.6696) (width 0.2) (layer "B.Cu") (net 4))
 (segment (start 99.4217 29.33) (end 100.7276 28.0241) (width 0.2) (layer "B.Cu") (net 4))
 (segment (start 140.7061 38.181) (end 141.0675 38.181) (width 0.2) (layer "B.Cu") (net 4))
 (segment (start 141.3839 31.6696) (end 141.3839 37.5032) (width 0.2) (layer "B.Cu") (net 4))
 (segment (start 141.3839 37.5032) (end 140.7061 38.181) (width 0.2) (layer "B.Cu") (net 4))
 (segment (start 141.0675 38.181) (end 140.7061 38.181) (width 0.2) (layer "B.Cu") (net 4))
 (segment (start 100.7276 28.0241) (end 137.7384 28.0241) (width 0.2) (layer "B.Cu") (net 4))
 (segment (start 140.3246 32.9516) (end 140.3246 32.9515) (width 0.2) (layer "F.Cu") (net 5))
 (segment (start 140.3246 32.9516) (end 140.3246 32.9515) (width 0.2) (layer "F.Cu") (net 5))
 (segment (start 142.9585 32.9515) (end 143.08 32.83) (width 0.2) (layer "F.Cu") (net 5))
 (segment (start 140.3246 32.9515) (end 142.9585 32.9515) (width 0.2) (layer "F.Cu") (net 5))
 (via (at 140.3246 32.9515) (size 0.6) (drill 0.3) (layers "F.Cu" "B.Cu") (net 5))
 (segment (start 140.3246 32.9516) (end 140.3246 32.9515) (width 0.2) (layer "B.Cu") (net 5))
 (segment (start 140.3246 32.9515) (end 140.3246 32.9516) (width 0.2) (layer "B.Cu") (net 5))
 (segment (start 98.12 34.33) (end 99.4984 32.9516) (width 0.2) (layer "B.Cu") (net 5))
 (segment (start 140.3246 32.9516) (end 140.3246 32.9515) (width 0.2) (layer "B.Cu") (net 5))
 (segment (start 99.4984 32.9516) (end 140.3246 32.9516) (width 0.2) (layer "B.Cu") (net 5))
 (segment (start 127.89 38.7898) (end 126.9598 38.7898) (width 0.2) (layer "F.Cu") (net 15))
 (segment (start 131.401 50.72676) (end 131.401 39.621) (width 0.2) (layer "F.Cu") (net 15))
 (segment (start 126.9598 38.7898) (end 126.08 37.91) (width 0.2) (layer "F.Cu") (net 15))
 (segment (start 131.401 39.621) (end 129.8 38.02) (width 0.2) (layer "F.Cu") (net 15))
 (segment (start 130.25 52.79) (end 130.25 51.87776) (width 0.2) (layer "F.Cu") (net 15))
 (segment (start 130.25 51.87776) (end 131.401 50.72676) (width 0.2) (layer "F.Cu") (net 15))
 (via (at 129.8 38.02) (size 0.6) (drill 0.3) (layers "F.Cu" "B.Cu") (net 15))
 (via (at 127.89 38.7898) (size 0.6) (drill 0.3) (layers "F.Cu" "B.Cu") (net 15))
 (segment (start 128.6598 38.02) (end 127.89 38.7898) (width 0.2) (layer "B.Cu") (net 15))
 (segment (start 129.8 38.02) (end 128.6598 38.02) (width 0.2) (layer "B.Cu") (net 15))
 (segment (start 140.116157 32.31) (end 140.959942 32.31) (width 0.2) (layer "F.Cu") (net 14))
 (segment (start 134.52 47.02) (end 139.7236 41.8164) (width 0.2) (layer "F.Cu") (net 14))
 (segment (start 130.25 50.25) (end 130.25 49.631) (width 0.2) (layer "F.Cu") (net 14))
 (segment (start 139.7236 32.702557) (end 140.116157 32.31) (width 0.2) (layer "F.Cu") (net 14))
 (segment (start 139.7236 41.8164) (end 139.7236 32.702557) (width 0.2) (layer "F.Cu") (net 14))
 (segment (start 130.25 49.631) (end 130.801 49.08) (width 0.2) (layer "F.Cu") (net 14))
 (segment (start 142.979942 30.29) (end 143.08 30.29) (width 0.2) (layer "F.Cu") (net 14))
 (segment (start 140.959942 32.31) (end 142.979942 30.29) (width 0.2) (layer "F.Cu") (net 14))
 (via (at 134.52 47.02) (size 0.6) (drill 0.3) (layers "F.Cu" "B.Cu") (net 14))
 (via (at 130.801 49.08) (size 0.6) (drill 0.3) (layers "F.Cu" "B.Cu") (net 14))
 (segment (start 132.46 49.08) (end 134.52 47.02) (width 0.2) (layer "B.Cu") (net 14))
 (segment (start 130.801 49.08) (end 132.46 49.08) (width 0.2) (layer "B.Cu") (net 14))
 (segment (start 129.099 54.179) (end 130.25 55.33) (width 0.2) (layer "F.Cu") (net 16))
 (segment (start 129.17 35.41) (end 129.099 35.481) (width 0.2) (layer "F.Cu") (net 16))
 (segment (start 129.099 35.481) (end 129.099 54.179) (width 0.2) (layer "F.Cu") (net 16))
 (segment (start 126.08 35.37) (end 127.89 35.37) (width 0.2) (layer "F.Cu") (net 16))
 (via (at 127.89 35.37) (size 0.6) (drill 0.3) (layers "F.Cu" "B.Cu") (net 16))
 (via (at 129.17 35.41) (size 0.6) (drill 0.3) (layers "F.Cu" "B.Cu") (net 16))
 (segment (start 129.13 35.37) (end 129.17 35.41) (width 0.2) (layer "B.Cu") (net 16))
 (segment (start 127.89 35.37) (end 129.13 35.37) (width 0.2) (layer "B.Cu") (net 16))
 (segment (start 101.71 40.5822) (end 103.21 42.0822) (width 0.2) (layer "B.Cu") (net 10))
 (segment (start 101.32 40.5822) (end 101.71 40.5822) (width 0.2) (layer "B.Cu") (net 10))
 (segment (start 103.21 42.0822) (end 108.44 42.0822) (width 0.2) (layer "B.Cu") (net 10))
 (segment (start 144.9189 37.0963) (end 144.9189 44.2899) (width 0.2) (layer "F.Cu") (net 11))
 (segment (start 145.2905 45.3395) (end 144.95 45.68) (width 0.2) (layer "F.Cu") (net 11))
 (segment (start 143.1926 35.37) (end 144.9189 37.0963) (width 0.2) (layer "F.Cu") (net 11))
 (segment (start 144.9189 44.2899) (end 143.93 45.2788) (width 0.2) (layer "F.Cu") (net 11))
 (segment (start 143.93 45.68) (end 144.95 45.68) (width 0.2) (layer "F.Cu") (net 11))
 (segment (start 145.2905 44.7691) (end 145.2905 45.3395) (width 0.2) (layer "F.Cu") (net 11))
 (segment (start 143.93 45.2788) (end 143.93 45.68) (width 0.2) (layer "F.Cu") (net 11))
 (segment (start 143.08 35.37) (end 143.1926 35.37) (width 0.2) (layer "F.Cu") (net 11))
 (via (at 145.2905 44.7691) (size 0.6) (drill 0.3) (layers "F.Cu" "B.Cu") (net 11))
 (segment (start 141.1036 40.5822) (end 145.2905 44.7691) (width 0.2) (layer "B.Cu") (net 11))
 (segment (start 113.64 40.5822) (end 141.1036 40.5822) (width 0.2) (layer "B.Cu") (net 11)))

